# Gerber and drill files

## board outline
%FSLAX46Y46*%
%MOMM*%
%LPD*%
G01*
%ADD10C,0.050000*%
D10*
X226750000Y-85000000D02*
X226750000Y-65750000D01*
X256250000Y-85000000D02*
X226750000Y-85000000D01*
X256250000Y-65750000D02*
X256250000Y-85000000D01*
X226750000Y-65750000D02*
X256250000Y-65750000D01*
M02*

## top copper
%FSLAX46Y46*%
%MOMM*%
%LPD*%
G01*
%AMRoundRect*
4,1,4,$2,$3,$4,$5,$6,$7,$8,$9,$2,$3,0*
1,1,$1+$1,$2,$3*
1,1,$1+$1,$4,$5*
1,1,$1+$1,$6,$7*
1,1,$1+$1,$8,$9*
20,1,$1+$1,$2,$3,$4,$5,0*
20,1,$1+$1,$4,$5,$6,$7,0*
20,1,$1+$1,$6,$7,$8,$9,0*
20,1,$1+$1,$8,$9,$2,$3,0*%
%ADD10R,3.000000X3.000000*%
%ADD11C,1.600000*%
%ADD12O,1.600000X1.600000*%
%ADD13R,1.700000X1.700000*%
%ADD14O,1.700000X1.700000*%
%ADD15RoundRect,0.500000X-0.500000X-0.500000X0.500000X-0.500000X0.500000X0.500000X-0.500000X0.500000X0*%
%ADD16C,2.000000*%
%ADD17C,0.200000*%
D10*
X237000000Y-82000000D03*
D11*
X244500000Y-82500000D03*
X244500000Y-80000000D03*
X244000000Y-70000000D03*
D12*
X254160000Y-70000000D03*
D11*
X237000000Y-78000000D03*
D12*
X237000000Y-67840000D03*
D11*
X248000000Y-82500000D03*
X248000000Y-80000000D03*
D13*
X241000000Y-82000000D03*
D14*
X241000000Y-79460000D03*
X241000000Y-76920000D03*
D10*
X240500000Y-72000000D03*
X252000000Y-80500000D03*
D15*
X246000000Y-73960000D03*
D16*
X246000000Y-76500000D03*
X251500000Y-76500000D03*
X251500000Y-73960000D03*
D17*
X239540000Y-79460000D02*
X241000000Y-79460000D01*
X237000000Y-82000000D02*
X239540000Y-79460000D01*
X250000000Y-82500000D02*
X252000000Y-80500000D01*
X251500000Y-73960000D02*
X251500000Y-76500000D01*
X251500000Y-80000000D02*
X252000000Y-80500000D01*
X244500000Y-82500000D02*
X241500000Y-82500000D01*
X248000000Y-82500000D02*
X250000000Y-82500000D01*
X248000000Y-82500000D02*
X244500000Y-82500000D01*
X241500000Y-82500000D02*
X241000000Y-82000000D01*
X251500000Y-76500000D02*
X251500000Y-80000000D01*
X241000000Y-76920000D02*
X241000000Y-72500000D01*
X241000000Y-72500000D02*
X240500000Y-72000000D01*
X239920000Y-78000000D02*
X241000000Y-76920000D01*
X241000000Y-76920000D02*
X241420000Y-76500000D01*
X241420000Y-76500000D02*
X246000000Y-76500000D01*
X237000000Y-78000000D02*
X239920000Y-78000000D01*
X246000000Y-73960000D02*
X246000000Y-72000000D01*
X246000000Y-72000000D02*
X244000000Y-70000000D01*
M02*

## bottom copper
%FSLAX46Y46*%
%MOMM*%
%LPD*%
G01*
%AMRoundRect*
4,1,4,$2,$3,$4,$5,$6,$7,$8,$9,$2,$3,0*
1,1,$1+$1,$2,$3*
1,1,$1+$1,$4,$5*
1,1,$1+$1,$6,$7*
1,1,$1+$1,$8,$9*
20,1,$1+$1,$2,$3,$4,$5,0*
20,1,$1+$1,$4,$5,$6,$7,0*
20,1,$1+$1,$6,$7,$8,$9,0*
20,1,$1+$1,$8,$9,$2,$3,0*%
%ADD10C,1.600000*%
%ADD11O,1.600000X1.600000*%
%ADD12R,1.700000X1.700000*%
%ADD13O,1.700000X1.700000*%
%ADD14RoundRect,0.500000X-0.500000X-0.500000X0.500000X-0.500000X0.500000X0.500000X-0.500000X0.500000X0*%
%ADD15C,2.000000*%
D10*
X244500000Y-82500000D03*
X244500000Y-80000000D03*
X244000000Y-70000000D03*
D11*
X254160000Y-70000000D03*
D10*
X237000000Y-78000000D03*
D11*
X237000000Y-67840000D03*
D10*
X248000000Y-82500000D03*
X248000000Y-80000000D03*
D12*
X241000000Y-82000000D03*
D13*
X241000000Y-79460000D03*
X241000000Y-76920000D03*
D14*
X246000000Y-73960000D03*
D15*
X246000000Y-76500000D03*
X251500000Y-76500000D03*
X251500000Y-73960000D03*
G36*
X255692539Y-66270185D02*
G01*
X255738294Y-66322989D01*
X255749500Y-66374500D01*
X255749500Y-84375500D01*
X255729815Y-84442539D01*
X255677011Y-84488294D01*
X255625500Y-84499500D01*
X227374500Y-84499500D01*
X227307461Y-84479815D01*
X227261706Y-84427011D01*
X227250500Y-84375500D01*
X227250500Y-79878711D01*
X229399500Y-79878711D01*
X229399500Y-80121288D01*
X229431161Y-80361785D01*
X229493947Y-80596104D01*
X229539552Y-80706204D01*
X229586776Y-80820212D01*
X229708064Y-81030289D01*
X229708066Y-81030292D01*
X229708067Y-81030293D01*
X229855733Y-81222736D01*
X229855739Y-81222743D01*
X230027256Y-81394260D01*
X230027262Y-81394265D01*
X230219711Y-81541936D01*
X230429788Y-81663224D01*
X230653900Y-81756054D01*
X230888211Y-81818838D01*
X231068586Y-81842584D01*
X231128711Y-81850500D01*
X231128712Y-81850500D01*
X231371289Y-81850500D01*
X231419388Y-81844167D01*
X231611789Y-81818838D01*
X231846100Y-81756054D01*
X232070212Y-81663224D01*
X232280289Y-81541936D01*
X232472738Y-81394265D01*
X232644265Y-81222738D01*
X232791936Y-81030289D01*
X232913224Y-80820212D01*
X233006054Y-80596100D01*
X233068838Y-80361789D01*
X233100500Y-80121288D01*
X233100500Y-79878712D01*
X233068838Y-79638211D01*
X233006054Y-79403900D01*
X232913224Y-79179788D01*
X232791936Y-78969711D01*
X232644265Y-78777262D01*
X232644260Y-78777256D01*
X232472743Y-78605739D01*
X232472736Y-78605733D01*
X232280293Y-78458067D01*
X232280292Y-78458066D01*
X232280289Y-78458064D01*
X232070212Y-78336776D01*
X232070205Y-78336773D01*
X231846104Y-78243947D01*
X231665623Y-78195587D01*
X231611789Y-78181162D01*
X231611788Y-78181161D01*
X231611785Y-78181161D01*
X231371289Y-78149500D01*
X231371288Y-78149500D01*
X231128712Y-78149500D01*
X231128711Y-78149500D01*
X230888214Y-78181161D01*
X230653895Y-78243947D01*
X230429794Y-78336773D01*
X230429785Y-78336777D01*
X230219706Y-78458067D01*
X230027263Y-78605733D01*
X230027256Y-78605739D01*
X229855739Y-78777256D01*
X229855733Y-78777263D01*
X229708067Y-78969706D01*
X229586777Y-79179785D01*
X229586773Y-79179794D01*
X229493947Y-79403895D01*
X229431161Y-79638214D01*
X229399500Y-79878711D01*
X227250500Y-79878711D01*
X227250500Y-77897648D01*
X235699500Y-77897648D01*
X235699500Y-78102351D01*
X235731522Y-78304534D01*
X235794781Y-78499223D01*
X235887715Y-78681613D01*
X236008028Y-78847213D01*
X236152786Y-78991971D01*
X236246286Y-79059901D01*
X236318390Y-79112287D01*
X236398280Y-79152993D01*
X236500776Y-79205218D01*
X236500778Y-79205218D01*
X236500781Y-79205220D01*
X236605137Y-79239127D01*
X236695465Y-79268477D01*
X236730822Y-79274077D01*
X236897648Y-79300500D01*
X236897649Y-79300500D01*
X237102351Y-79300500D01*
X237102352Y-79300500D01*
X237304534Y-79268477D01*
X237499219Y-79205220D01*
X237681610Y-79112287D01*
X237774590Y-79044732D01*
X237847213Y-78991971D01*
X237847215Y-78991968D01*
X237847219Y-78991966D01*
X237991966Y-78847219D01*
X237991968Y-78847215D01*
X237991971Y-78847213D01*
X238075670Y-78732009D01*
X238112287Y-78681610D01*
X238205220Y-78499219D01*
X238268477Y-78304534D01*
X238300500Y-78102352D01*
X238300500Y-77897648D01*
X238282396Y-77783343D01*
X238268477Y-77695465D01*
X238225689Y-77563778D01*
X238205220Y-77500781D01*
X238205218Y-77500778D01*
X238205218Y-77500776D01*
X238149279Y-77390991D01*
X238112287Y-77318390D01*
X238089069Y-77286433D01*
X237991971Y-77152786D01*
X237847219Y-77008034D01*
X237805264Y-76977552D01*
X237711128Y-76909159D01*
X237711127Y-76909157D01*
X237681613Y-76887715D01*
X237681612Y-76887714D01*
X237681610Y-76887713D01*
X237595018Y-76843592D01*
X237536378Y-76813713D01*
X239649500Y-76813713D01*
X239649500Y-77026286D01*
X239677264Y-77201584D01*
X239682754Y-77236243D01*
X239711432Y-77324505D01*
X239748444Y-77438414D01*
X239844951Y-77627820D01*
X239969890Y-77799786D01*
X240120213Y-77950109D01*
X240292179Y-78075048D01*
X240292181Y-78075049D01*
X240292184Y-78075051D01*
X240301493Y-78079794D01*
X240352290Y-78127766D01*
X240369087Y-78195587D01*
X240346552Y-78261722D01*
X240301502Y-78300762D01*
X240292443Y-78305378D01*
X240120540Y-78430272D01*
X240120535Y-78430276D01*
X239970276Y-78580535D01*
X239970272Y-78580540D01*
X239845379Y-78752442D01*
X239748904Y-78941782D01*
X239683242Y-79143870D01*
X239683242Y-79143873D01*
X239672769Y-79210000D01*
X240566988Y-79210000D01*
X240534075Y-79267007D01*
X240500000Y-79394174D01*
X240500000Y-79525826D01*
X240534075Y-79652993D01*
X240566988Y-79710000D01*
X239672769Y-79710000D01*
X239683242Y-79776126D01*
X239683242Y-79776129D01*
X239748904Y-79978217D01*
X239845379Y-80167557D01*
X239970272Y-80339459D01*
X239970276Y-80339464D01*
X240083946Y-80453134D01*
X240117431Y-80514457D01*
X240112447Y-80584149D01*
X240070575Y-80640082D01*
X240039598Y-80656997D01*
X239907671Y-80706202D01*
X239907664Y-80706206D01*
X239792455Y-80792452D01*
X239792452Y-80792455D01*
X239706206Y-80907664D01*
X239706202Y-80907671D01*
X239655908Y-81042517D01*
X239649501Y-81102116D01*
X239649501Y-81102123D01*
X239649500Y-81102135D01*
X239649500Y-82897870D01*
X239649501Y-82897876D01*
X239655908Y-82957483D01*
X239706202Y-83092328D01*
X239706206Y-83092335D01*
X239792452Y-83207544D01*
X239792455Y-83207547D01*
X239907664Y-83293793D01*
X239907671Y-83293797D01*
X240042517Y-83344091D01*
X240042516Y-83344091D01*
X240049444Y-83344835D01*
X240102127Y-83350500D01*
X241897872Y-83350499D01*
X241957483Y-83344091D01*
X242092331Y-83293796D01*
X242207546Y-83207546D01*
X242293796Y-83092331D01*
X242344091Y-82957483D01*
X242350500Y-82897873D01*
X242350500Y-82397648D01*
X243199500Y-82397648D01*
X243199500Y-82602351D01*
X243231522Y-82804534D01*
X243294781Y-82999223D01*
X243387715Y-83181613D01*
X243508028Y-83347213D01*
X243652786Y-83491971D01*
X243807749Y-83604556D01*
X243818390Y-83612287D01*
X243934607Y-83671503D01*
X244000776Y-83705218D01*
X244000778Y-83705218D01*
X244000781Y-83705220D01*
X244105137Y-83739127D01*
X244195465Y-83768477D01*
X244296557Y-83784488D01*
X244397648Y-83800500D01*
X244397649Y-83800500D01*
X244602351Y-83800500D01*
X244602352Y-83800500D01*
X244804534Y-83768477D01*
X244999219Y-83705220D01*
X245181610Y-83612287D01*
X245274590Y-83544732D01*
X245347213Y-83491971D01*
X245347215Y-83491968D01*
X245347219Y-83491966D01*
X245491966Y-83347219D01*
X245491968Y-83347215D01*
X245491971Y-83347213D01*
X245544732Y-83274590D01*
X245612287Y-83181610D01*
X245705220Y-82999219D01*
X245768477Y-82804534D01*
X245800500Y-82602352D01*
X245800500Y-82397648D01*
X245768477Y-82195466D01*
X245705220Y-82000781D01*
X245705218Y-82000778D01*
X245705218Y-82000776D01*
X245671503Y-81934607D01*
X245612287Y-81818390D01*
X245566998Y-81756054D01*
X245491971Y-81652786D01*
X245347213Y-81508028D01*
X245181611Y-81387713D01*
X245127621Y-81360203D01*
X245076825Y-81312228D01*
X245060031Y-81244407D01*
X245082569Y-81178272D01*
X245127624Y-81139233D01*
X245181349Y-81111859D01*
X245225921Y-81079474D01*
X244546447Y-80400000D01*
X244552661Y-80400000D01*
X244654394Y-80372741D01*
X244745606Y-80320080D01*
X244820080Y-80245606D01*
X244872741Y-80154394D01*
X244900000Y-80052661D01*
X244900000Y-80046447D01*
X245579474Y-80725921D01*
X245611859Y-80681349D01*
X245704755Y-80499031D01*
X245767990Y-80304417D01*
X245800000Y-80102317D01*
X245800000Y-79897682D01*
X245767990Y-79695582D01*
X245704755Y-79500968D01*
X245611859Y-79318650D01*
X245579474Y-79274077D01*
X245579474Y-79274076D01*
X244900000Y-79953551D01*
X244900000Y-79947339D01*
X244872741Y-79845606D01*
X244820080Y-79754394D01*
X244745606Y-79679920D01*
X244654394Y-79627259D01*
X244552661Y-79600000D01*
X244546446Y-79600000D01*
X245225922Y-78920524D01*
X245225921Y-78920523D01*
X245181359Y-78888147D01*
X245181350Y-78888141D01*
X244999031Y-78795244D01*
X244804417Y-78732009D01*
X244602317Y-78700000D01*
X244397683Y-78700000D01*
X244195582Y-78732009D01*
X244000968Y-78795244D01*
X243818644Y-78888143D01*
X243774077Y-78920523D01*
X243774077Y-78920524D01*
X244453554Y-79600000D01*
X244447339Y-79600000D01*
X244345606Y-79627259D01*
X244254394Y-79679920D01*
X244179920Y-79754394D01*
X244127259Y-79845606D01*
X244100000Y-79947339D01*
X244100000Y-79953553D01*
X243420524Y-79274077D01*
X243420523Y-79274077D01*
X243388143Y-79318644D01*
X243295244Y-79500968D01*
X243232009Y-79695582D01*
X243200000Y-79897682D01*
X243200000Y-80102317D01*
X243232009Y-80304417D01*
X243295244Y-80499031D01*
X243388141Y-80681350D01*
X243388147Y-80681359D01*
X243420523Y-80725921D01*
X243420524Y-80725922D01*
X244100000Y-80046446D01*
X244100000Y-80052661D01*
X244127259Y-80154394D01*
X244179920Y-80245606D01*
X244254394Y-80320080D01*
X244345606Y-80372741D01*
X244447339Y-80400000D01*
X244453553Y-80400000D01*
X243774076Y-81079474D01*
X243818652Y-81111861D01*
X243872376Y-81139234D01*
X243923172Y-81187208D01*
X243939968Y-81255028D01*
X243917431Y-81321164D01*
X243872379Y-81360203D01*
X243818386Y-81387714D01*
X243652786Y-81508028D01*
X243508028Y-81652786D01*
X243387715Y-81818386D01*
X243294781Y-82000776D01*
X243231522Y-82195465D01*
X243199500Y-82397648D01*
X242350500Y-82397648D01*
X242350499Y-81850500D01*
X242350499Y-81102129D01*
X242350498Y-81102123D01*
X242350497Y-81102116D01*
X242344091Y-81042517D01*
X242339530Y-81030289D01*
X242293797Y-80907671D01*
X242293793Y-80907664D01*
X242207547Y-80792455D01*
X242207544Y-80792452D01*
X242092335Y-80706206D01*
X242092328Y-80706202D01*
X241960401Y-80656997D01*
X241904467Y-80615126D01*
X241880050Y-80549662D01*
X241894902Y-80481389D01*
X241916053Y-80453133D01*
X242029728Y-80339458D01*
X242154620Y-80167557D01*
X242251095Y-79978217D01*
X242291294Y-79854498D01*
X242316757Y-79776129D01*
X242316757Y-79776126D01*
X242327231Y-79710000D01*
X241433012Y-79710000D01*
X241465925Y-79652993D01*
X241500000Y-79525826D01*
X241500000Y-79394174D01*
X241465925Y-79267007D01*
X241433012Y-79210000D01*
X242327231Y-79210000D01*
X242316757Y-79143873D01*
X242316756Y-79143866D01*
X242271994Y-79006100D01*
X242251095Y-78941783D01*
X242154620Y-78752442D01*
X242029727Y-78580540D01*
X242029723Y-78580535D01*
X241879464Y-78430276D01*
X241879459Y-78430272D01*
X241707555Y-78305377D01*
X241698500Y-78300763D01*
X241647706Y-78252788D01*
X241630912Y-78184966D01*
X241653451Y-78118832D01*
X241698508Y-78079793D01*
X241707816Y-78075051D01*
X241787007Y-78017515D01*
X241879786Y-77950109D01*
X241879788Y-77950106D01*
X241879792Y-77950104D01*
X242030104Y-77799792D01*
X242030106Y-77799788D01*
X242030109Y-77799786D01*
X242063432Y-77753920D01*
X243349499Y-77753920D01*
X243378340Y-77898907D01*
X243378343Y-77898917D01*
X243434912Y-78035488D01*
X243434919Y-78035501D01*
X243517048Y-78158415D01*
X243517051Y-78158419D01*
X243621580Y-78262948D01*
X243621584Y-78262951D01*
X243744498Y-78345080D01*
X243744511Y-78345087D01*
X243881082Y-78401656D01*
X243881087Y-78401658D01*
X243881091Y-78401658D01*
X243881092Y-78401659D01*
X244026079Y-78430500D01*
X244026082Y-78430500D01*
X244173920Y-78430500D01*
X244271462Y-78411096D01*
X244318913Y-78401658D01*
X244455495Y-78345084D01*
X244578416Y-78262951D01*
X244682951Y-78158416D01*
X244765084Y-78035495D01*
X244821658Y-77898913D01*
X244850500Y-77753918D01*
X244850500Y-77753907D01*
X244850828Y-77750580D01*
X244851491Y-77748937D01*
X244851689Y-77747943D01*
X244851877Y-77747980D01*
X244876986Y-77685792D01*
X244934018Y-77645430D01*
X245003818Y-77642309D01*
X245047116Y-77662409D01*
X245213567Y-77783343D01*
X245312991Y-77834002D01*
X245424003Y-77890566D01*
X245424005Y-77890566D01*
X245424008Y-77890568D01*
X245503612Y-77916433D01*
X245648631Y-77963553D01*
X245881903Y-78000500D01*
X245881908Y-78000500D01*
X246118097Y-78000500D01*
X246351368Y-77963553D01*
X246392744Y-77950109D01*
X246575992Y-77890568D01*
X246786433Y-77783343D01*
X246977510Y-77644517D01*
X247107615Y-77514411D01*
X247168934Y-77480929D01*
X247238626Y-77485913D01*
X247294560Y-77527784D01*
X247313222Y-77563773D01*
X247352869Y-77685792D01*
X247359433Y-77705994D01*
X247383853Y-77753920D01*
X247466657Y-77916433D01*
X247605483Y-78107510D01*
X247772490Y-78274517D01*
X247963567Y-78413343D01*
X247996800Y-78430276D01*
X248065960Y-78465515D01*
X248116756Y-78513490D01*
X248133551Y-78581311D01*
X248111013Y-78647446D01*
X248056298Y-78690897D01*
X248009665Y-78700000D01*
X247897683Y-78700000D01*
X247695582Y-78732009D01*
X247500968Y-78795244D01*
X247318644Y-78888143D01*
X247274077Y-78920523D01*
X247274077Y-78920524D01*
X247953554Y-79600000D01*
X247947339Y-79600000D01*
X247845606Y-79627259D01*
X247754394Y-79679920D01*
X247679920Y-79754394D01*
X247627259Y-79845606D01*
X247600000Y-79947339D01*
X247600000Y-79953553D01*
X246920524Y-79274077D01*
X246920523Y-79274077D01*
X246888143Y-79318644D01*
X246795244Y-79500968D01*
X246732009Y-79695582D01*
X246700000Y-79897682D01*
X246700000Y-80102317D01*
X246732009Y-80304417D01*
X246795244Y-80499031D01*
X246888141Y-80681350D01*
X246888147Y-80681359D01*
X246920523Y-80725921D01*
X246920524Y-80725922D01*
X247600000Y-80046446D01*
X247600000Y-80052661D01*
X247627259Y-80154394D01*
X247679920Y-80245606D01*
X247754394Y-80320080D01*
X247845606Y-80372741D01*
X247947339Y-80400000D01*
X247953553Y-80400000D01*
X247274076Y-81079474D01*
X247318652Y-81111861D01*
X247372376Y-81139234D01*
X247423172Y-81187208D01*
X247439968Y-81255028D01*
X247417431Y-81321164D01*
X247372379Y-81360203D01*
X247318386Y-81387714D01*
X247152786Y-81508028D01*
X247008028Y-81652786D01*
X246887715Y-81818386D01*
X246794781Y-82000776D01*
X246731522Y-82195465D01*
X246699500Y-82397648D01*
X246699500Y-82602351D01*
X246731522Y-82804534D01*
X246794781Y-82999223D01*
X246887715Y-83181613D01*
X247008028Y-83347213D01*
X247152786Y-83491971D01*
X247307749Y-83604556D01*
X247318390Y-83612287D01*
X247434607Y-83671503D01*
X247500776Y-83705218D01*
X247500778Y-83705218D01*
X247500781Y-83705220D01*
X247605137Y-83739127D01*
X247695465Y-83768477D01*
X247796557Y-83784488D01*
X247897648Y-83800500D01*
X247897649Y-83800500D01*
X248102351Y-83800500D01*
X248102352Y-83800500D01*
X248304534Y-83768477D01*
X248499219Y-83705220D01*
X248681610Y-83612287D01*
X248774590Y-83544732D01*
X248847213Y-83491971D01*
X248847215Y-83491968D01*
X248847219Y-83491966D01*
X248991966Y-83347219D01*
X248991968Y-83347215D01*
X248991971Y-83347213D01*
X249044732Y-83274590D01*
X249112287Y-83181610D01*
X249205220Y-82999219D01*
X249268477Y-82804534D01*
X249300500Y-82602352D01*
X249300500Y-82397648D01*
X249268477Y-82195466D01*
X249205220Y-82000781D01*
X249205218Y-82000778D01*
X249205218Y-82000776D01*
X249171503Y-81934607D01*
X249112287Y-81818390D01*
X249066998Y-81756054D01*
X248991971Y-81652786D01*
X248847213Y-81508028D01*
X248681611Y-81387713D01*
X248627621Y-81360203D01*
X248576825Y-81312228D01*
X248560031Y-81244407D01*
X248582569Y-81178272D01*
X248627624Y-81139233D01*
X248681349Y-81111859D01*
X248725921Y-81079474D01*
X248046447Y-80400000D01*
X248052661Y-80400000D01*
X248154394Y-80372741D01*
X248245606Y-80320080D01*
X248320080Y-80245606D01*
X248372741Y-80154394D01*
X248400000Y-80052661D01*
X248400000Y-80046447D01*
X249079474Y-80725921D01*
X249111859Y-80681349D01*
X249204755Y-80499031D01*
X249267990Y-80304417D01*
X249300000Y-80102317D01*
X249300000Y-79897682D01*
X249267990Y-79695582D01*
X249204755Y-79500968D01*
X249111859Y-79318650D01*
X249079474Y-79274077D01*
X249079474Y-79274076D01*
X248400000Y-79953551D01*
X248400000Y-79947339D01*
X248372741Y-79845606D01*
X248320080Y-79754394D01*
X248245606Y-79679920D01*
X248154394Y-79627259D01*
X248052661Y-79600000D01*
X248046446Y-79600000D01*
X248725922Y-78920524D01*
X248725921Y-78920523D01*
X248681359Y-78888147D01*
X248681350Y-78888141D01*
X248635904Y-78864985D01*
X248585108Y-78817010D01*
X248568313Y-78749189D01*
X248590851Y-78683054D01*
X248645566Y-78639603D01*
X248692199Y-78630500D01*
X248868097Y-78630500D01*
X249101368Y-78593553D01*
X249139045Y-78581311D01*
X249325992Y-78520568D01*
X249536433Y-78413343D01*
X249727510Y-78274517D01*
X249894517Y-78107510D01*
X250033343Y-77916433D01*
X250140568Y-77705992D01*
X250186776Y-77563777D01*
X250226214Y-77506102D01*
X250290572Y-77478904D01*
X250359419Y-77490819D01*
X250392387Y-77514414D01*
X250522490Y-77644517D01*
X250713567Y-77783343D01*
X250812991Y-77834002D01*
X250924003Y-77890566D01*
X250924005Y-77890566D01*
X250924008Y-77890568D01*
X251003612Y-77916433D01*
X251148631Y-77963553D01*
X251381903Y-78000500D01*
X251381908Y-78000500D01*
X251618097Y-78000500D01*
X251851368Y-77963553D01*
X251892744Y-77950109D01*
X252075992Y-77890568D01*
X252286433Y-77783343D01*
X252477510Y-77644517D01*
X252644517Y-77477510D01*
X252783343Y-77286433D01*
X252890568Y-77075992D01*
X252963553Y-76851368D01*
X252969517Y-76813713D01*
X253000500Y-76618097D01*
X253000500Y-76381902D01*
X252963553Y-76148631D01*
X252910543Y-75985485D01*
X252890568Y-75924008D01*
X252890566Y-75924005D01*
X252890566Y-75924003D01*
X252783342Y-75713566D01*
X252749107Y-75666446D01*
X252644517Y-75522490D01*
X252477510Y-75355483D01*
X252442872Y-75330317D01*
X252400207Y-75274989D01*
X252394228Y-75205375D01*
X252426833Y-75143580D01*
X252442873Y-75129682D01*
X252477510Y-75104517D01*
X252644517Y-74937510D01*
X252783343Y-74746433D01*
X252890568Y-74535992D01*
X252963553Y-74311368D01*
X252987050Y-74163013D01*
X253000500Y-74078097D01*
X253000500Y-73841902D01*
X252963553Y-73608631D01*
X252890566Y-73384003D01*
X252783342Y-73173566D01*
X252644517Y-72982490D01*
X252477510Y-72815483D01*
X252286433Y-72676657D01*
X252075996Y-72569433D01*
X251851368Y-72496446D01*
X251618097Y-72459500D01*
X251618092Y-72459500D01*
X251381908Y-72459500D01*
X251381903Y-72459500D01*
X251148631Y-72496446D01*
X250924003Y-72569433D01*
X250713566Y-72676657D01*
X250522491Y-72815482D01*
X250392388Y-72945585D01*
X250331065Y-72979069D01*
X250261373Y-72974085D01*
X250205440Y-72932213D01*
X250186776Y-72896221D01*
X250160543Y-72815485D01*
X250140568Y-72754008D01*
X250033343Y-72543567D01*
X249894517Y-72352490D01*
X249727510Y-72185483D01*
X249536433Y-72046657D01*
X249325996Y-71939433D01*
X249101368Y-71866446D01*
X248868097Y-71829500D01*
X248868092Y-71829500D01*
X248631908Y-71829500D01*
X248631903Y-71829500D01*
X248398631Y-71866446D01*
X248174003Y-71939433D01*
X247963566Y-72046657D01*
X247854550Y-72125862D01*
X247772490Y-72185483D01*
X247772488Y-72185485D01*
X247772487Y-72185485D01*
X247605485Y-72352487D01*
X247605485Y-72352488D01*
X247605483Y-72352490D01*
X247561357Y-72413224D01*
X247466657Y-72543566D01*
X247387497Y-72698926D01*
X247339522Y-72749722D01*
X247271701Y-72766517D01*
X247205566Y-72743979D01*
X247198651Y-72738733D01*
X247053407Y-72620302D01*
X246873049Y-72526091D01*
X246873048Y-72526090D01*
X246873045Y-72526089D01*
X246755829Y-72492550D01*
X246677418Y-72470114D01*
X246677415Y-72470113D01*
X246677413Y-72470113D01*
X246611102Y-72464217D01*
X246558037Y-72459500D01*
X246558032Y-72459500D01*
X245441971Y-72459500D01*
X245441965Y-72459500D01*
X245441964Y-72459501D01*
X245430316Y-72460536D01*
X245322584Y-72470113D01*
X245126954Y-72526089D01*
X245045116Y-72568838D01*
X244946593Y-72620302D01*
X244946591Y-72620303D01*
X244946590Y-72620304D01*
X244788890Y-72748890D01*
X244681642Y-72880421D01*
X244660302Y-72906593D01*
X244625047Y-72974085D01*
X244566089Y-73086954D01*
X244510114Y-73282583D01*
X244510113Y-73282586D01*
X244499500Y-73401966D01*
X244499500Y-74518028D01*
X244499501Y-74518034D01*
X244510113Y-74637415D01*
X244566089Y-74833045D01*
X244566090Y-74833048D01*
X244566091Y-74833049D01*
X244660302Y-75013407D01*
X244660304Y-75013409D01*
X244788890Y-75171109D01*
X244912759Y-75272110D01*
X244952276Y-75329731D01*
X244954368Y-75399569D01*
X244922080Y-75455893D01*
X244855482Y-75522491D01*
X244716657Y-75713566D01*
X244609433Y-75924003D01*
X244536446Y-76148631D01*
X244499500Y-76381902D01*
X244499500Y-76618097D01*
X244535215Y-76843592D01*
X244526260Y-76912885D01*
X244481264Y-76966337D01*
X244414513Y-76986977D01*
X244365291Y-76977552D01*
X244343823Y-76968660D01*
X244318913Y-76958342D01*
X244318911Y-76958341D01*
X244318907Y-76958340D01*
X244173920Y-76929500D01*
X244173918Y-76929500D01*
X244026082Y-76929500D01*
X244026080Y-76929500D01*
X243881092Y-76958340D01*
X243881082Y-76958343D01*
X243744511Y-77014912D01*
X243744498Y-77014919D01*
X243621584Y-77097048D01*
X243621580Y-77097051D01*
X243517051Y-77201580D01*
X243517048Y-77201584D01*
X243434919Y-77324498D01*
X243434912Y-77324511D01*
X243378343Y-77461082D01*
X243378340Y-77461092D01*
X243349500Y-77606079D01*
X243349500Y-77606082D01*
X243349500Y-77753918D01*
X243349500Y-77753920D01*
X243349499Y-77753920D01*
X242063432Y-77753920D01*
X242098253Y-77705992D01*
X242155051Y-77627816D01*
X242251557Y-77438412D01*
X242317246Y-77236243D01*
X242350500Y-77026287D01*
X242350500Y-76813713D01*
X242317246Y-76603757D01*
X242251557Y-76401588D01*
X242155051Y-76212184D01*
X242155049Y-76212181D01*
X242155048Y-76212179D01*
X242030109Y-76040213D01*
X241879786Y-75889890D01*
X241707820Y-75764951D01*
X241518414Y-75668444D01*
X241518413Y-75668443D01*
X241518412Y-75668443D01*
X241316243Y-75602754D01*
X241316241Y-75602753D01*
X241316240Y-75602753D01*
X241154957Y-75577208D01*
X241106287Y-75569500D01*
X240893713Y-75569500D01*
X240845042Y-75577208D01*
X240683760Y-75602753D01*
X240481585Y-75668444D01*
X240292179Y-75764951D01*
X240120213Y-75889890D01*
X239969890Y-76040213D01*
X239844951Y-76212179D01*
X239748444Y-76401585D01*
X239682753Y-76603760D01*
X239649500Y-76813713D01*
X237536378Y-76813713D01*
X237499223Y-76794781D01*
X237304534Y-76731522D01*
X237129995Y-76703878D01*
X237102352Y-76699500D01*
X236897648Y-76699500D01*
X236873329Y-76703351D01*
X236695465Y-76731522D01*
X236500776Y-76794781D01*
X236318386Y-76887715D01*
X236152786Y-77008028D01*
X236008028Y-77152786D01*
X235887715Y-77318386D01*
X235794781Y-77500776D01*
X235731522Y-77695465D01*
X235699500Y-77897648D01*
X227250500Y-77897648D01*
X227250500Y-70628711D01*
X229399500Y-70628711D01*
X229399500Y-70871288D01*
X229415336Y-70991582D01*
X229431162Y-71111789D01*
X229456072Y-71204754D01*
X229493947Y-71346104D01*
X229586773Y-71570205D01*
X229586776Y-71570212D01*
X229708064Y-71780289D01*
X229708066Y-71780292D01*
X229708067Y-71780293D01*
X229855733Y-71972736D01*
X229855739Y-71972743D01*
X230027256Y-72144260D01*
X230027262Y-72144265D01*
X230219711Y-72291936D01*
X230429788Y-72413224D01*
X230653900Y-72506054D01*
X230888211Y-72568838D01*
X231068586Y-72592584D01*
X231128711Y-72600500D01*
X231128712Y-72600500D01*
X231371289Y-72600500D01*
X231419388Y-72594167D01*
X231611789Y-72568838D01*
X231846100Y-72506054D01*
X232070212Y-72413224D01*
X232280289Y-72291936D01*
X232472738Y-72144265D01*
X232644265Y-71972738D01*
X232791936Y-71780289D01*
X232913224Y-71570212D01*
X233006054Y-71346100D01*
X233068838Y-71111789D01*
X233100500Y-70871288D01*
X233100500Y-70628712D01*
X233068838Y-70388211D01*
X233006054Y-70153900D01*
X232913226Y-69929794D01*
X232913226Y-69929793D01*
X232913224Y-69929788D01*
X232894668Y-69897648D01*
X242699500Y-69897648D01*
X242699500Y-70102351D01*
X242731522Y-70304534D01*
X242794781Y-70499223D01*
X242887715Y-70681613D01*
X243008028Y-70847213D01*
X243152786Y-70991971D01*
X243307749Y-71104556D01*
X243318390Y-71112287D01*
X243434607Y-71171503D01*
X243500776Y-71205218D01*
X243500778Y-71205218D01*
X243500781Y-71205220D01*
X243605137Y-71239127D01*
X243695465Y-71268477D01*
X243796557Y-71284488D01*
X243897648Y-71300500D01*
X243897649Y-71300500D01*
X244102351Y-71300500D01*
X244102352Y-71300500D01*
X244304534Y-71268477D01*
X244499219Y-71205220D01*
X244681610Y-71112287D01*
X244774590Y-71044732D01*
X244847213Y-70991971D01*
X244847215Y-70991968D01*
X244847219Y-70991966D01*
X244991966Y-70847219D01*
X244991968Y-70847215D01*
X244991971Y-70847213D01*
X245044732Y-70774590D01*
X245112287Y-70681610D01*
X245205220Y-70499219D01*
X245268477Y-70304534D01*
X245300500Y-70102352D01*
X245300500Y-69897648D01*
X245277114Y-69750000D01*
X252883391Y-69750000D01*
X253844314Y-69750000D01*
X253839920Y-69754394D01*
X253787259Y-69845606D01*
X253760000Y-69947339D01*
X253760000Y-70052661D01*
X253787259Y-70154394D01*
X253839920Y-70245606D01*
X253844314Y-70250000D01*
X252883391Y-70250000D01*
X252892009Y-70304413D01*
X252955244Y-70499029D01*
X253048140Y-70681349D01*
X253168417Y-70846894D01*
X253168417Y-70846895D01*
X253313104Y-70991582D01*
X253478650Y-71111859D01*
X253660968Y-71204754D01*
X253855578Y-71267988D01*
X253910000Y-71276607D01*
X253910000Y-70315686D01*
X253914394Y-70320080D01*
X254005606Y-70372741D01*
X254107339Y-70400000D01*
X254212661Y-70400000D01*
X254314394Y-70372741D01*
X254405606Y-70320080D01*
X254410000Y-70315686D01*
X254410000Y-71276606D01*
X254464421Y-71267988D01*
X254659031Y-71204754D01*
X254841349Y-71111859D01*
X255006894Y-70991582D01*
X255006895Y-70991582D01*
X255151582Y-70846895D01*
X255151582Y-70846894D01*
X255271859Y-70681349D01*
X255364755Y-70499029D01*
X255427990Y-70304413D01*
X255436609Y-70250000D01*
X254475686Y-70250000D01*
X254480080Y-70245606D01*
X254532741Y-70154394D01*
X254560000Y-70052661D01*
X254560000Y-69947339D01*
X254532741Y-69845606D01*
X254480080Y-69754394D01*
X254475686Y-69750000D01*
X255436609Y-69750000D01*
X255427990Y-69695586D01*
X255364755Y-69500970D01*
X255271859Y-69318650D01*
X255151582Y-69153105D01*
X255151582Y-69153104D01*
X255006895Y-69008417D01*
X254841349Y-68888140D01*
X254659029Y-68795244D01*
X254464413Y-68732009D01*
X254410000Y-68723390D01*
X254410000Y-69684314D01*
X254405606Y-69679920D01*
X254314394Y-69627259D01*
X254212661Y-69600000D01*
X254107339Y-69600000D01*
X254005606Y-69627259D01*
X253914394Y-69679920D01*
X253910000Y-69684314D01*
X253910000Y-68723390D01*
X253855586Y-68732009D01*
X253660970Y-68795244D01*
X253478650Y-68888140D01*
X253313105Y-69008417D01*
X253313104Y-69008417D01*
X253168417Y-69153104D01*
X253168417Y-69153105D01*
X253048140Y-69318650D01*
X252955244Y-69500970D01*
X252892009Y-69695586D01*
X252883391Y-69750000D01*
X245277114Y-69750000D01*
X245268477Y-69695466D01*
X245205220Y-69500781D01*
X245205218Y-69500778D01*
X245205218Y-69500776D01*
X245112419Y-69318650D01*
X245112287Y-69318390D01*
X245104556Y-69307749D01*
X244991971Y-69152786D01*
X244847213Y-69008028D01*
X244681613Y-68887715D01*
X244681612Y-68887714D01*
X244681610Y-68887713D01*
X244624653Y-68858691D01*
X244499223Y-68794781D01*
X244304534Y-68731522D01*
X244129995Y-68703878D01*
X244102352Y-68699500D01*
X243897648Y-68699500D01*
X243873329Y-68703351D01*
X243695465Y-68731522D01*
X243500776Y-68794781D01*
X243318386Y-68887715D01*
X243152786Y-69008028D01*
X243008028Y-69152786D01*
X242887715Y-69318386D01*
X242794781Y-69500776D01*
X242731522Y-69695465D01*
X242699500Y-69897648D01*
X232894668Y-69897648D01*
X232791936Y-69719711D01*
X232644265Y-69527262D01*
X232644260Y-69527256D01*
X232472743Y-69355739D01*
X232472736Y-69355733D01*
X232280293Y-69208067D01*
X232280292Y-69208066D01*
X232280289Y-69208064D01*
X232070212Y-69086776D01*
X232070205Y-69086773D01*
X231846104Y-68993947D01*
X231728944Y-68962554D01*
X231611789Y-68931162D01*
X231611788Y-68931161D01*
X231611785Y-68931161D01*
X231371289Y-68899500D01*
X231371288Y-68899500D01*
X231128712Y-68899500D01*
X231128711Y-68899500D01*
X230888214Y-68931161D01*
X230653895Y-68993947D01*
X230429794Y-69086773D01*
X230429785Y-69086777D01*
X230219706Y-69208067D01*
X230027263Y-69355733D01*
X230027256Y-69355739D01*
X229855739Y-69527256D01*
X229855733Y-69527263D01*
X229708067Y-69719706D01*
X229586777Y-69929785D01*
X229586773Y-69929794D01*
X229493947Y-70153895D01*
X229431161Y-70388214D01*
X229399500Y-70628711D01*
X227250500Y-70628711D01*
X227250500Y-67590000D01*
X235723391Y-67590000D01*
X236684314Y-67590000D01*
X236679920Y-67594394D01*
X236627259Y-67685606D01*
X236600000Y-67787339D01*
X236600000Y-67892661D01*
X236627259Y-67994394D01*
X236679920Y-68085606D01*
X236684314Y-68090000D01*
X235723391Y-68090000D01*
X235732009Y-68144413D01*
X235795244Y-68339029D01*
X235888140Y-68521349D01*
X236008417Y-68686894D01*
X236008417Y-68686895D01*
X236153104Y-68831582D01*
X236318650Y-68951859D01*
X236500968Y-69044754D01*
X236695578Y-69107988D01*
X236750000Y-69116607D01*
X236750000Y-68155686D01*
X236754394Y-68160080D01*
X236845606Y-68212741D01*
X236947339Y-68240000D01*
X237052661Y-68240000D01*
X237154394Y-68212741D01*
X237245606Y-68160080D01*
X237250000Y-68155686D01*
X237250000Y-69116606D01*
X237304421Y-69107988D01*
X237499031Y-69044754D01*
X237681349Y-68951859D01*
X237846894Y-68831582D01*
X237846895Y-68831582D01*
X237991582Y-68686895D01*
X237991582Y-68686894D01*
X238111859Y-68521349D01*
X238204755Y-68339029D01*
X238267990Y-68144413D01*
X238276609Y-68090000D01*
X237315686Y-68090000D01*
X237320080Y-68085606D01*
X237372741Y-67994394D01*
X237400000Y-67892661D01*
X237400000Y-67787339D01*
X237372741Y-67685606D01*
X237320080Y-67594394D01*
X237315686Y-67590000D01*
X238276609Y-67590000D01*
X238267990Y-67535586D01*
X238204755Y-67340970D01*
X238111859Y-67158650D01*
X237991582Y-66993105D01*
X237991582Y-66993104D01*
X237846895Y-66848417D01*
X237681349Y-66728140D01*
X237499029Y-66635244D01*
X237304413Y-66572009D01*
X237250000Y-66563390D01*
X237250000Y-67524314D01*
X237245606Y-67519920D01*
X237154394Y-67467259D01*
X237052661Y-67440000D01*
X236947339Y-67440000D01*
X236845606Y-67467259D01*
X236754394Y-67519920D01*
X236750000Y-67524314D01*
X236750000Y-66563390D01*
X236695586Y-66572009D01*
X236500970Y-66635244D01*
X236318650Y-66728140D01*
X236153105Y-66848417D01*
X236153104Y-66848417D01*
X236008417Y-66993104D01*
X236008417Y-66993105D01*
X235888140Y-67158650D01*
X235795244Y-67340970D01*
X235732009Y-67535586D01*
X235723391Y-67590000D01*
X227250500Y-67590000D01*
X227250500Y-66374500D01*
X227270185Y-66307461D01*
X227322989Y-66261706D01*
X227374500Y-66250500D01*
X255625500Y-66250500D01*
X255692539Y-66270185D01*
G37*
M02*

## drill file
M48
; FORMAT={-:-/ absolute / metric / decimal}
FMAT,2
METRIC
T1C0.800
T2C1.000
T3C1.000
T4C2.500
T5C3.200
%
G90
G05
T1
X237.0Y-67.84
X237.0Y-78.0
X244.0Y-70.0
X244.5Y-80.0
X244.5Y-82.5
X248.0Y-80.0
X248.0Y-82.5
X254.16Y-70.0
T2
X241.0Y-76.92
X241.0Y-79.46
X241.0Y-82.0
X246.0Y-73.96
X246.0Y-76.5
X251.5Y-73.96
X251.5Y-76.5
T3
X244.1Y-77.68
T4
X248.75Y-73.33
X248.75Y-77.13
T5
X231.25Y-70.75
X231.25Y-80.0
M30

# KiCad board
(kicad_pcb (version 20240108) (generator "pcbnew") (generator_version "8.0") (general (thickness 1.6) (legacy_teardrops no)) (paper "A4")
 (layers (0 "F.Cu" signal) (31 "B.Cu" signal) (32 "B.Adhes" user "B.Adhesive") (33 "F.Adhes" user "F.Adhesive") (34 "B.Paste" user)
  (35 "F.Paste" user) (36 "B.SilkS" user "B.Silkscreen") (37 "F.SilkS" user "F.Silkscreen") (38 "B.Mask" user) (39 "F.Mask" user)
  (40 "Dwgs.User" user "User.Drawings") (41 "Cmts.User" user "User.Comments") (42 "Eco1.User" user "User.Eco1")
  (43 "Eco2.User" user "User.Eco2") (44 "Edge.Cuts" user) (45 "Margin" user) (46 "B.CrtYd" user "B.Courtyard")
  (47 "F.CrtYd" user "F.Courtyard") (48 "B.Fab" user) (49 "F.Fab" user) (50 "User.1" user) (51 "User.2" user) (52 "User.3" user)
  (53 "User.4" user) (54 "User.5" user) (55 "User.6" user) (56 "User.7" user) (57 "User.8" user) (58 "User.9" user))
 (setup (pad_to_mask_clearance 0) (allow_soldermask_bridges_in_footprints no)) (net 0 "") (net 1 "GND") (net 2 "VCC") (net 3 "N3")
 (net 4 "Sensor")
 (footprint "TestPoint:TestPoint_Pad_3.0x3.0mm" (layer "F.Cu") (at 237 82)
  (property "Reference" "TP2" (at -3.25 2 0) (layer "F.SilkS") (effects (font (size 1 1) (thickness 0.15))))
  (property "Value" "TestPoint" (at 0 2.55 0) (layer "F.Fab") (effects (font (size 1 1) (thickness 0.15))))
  (pad "1" smd rect (at 0 0) (size 3 3) (layers "F.Cu" "F.Mask") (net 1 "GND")))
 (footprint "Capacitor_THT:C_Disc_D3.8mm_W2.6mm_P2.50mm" (layer "F.Cu") (at 244.5 82.5 90)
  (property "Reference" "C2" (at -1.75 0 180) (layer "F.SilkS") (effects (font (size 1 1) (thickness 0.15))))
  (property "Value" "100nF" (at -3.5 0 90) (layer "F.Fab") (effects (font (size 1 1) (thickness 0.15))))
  (pad "1" thru_hole circle (at 0 0 90) (size 1.6 1.6) (drill 0.8) (layers "*.Cu" "*.Mask") (remove_unused_layers no) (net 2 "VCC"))
  (pad "2" thru_hole circle (at 2.5 0 90) (size 1.6 1.6) (drill 0.8) (layers "*.Cu" "*.Mask") (remove_unused_layers no) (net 1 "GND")))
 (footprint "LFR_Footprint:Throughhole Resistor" (layer "F.Cu") (at 244 70)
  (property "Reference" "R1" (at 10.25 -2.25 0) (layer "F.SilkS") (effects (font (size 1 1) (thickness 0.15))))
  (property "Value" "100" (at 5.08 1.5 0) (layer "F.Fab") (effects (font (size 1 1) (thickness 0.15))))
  (pad "1" thru_hole circle (at 0 0) (size 1.6 1.6) (drill 0.8) (layers "*.Cu" "*.Mask") (remove_unused_layers no) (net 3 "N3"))
  (pad "2" thru_hole oval (at 10.16 0) (size 1.6 1.6) (drill 0.8) (layers "*.Cu" "*.Mask") (remove_unused_layers no) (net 1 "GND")))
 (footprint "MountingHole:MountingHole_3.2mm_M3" (layer "F.Cu") (at 231.25 70.75)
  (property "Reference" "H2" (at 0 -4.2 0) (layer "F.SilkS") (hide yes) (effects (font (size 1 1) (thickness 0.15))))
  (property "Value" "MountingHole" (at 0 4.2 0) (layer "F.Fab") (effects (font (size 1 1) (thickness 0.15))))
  (pad "" np_thru_hole circle (at 0 0) (size 3.2 3.2) (drill 3.2) (layers "*.Cu" "*.Mask")))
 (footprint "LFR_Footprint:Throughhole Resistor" (layer "F.Cu") (at 237 78 90)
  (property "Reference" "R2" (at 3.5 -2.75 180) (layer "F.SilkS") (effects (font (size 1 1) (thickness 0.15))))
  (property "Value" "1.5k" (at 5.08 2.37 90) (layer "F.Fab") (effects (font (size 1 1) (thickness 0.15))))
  (pad "1" thru_hole circle (at 0 0 90) (size 1.6 1.6) (drill 0.8) (layers "*.Cu" "*.Mask") (remove_unused_layers no) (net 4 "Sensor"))
  (pad "2" thru_hole oval (at 10.16 0 90) (size 1.6 1.6) (drill 0.8) (layers "*.Cu" "*.Mask") (remove_unused_layers no) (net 1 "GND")))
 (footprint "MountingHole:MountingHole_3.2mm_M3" (layer "F.Cu") (at 231.25 80)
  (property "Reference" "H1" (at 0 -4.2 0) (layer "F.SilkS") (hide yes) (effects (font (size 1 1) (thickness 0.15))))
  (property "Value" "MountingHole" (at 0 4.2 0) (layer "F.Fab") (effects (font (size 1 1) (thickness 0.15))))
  (pad "" np_thru_hole circle (at 0 0) (size 3.2 3.2) (drill 3.2) (layers "*.Cu" "*.Mask")))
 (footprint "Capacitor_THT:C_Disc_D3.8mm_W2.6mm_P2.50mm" (layer "F.Cu") (at 248 82.5 90)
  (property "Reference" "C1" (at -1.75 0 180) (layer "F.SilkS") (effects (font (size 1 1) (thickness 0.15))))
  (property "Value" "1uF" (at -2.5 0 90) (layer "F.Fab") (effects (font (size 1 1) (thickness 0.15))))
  (pad "1" thru_hole circle (at 0 0 90) (size 1.6 1.6) (drill 0.8) (layers "*.Cu" "*.Mask") (remove_unused_layers no) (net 2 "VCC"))
  (pad "2" thru_hole circle (at 2.5 0 90) (size 1.6 1.6) (drill 0.8) (layers "*.Cu" "*.Mask") (remove_unused_layers no) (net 1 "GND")))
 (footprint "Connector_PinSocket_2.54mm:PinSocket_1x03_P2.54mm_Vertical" (layer "F.Cu") (at 241 82 180)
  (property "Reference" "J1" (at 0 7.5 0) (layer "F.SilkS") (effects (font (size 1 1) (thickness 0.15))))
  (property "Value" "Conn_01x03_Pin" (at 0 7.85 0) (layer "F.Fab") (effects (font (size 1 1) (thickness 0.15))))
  (pad "1" thru_hole rect (at 0 0 180) (size 1.7 1.7) (drill 1) (layers "*.Cu" "*.Mask") (remove_unused_layers no) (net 2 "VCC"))
  (pad "2" thru_hole oval (at 0 2.54 180) (size 1.7 1.7) (drill 1) (layers "*.Cu" "*.Mask") (remove_unused_layers no) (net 1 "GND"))
  (pad "3" thru_hole oval (at 0 5.08 180) (size 1.7 1.7) (drill 1) (layers "*.Cu" "*.Mask") (remove_unused_layers no) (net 4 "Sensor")))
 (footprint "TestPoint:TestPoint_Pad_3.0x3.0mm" (layer "F.Cu") (at 240.5 72)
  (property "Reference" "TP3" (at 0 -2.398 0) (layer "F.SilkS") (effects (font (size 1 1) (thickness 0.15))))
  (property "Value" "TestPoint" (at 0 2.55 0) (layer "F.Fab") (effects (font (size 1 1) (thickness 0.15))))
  (pad "1" smd rect (at 0 0) (size 3 3) (layers "F.Cu" "F.Mask") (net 4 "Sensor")))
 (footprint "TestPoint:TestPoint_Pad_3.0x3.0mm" (layer "F.Cu") (at 252 80.5)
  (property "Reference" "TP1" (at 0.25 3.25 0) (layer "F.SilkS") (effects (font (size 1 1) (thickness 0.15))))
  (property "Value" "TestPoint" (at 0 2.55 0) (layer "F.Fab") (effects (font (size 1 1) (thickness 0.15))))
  (pad "1" smd rect (at 0 0) (size 3 3) (layers "F.Cu" "F.Mask") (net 2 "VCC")))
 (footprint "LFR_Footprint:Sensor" (layer "F.Cu") (at 246 73.96)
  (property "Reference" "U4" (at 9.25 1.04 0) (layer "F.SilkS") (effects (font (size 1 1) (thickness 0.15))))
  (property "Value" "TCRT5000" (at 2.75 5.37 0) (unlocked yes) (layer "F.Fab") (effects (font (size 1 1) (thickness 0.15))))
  (pad "" np_thru_hole circle (at -1.9 3.72) (size 1 1) (drill 1) (layers "F&B.Cu" "*.Mask"))
  (pad "" np_thru_hole circle (at 2.75 -0.63) (size 2.5 2.5) (drill 2.5) (layers "F&B.Cu" "*.Mask"))
  (pad "" np_thru_hole circle (at 2.75 3.17) (size 2.5 2.5) (drill 2.5) (layers "F&B.Cu" "*.Mask"))
  (pad "1" thru_hole roundrect (at 0 0) (size 2 2) (drill 1) (layers "*.Cu" "*.Mask") (remove_unused_layers no) (roundrect_rratio 0.25)
   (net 3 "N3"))
  (pad "2" thru_hole circle (at 0 2.54) (size 2 2) (drill 1) (layers "*.Cu" "*.Mask") (remove_unused_layers no) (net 4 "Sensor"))
  (pad "3" thru_hole circle (at 5.5 2.54) (size 2 2) (drill 1) (layers "*.Cu" "*.Mask") (remove_unused_layers no) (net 2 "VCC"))
  (pad "4" thru_hole circle (at 5.5 0) (size 2 2) (drill 1) (layers "*.Cu" "*.Mask") (remove_unused_layers no) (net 2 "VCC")))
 (gr_line (start 226.75 85) (end 226.75 65.75) (stroke (width 0.05) (type default)) (layer "Edge.Cuts"))
 (gr_line (start 256.25 85) (end 226.75 85) (stroke (width 0.05) (type default)) (layer "Edge.Cuts"))
 (gr_line (start 256.25 65.75) (end 256.25 85) (stroke (width 0.05) (type default)) (layer "Edge.Cuts"))
 (gr_line (start 226.75 65.75) (end 256.25 65.75) (stroke (width 0.05) (type default)) (layer "Edge.Cuts"))
 (segment (start 239.54 79.46) (end 241 79.46) (width 0.2) (layer "F.Cu") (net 1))
 (segment (start 237 82) (end 239.54 79.46) (width 0.2) (layer "F.Cu") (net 1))
 (segment (start 250 82.5) (end 252 80.5) (width 0.2) (layer "F.Cu") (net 2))
 (segment (start 251.5 73.96) (end 251.5 76.5) (width 0.2) (layer "F.Cu") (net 2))
 (segment (start 251.5 80) (end 252 80.5) (width 0.2) (layer "F.Cu") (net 2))
 (segment (start 244.5 82.5) (end 241.5 82.5) (width 0.2) (layer "F.Cu") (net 2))
 (segment (start 248 82.5) (end 250 82.5) (width 0.2) (layer "F.Cu") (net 2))
 (segment (start 248 82.5) (end 244.5 82.5) (width 0.2) (layer "F.Cu") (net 2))
 (segment (start 241.5 82.5) (end 241 82) (width 0.2) (layer "F.Cu") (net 2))
 (segment (start 251.5 76.5) (end 251.5 80) (width 0.2) (layer "F.Cu") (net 2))
 (segment (start 241 76.92) (end 241 72.5) (width 0.2) (layer "F.Cu") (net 4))
 (segment (start 241 72.5) (end 240.5 72) (width 0.2) (layer "F.Cu") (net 4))
 (segment (start 239.92 78) (end 241 76.92) (width 0.2) (layer "F.Cu") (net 4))
 (segment (start 241 76.92) (end 241.42 76.5) (width 0.2) (layer "F.Cu") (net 4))
 (segment (start 241.42 76.5) (end 246 76.5) (width 0.2) (layer "F.Cu") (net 4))
 (segment (start 237 78) (end 239.92 78) (width 0.2) (layer "F.Cu") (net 4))
 (segment (start 246 73.96) (end 246 72) (width 0.2) (layer "F.Cu") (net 3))
 (segment (start 246 72) (end 244 70) (width 0.2) (layer "F.Cu") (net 3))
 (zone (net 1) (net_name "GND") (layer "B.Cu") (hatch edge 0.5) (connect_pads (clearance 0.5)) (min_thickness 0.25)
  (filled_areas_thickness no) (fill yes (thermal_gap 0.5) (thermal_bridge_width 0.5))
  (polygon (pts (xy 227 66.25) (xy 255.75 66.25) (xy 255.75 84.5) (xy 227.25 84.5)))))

